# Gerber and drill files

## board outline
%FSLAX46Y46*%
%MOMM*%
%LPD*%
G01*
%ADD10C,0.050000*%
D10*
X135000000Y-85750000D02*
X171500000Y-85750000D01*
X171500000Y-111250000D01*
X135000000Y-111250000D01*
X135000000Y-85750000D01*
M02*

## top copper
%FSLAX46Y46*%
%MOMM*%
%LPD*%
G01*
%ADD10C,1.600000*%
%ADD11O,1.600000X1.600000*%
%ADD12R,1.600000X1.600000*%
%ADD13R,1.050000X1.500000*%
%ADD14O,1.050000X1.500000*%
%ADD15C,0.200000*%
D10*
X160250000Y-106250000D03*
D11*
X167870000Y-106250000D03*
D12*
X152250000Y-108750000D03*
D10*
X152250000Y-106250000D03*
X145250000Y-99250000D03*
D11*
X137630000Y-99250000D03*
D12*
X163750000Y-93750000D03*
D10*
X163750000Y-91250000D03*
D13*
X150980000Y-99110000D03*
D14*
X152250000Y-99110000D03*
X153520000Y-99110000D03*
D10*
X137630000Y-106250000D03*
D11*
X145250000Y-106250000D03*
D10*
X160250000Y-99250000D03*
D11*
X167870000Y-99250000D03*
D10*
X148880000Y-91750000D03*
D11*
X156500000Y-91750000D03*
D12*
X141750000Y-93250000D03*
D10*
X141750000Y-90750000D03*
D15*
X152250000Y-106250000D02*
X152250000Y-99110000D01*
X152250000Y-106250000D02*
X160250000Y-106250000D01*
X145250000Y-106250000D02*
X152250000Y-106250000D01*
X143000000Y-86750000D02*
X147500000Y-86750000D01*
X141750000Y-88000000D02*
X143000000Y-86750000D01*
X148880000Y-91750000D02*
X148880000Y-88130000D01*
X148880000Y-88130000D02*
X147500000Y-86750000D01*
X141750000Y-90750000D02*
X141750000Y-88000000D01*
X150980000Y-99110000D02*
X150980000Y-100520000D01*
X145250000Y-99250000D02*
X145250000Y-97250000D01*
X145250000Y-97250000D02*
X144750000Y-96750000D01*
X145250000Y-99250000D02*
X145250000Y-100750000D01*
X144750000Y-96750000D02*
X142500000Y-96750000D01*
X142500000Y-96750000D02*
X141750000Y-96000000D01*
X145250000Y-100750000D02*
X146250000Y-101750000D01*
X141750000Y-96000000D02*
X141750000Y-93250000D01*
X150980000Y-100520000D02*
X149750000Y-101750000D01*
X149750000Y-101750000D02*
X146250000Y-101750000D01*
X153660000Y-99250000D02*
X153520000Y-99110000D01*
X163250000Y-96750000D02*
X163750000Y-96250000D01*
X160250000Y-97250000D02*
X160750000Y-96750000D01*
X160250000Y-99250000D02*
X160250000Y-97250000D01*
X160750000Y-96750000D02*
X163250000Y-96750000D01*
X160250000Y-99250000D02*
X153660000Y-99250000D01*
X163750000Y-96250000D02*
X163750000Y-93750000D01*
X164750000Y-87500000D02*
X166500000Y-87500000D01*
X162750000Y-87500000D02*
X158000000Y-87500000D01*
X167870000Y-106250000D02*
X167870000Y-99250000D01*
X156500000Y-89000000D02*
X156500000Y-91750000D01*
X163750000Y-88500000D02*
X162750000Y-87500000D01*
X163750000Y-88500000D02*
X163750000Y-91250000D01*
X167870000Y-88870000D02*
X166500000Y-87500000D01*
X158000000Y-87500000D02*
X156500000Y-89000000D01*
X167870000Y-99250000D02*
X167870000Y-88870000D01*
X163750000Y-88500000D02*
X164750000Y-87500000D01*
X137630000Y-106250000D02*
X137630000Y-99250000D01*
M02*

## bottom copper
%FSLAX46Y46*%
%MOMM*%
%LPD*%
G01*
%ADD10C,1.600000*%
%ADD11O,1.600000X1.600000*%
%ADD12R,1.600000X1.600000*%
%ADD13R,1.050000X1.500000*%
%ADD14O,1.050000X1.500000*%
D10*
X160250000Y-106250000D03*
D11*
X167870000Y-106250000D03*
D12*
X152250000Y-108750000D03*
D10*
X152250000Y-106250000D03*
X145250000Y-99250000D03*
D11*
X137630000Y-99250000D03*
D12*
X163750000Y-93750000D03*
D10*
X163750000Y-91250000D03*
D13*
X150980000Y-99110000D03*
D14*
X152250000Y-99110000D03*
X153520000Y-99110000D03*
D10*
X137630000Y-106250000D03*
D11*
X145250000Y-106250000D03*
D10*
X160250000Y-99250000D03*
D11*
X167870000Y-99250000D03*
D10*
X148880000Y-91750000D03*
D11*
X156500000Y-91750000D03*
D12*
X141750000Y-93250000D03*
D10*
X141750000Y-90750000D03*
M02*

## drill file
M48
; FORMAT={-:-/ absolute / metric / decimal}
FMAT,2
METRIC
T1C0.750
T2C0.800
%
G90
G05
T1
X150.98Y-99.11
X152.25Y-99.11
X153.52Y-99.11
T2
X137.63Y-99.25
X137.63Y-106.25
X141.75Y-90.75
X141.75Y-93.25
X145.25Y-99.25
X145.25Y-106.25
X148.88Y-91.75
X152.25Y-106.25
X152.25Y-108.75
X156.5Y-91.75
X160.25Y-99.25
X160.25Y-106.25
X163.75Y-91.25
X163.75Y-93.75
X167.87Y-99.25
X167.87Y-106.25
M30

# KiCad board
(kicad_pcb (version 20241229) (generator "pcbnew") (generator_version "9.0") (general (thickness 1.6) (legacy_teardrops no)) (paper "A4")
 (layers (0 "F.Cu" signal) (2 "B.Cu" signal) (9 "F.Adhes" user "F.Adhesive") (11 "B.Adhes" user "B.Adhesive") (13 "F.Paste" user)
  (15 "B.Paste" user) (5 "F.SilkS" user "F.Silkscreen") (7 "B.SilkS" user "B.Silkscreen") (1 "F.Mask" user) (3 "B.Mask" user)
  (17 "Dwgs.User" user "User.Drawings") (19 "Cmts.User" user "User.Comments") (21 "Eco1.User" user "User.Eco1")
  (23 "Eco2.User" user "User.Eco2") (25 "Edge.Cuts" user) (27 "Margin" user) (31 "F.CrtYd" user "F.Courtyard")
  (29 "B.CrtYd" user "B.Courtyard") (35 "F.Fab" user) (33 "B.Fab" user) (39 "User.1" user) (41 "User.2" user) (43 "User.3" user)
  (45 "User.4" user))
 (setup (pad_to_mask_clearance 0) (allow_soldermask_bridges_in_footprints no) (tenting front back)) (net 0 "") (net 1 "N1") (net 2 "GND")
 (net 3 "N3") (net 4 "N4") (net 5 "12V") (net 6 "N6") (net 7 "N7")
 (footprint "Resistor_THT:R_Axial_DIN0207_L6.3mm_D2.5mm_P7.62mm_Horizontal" (layer "F.Cu") (at 160.25 106.25)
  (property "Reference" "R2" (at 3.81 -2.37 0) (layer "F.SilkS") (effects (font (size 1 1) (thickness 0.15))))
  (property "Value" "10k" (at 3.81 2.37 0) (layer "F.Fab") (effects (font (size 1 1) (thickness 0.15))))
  (pad "1" thru_hole circle (at 0 0) (size 1.6 1.6) (drill 0.8) (layers "*.Cu" "*.Mask") (remove_unused_layers no) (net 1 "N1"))
  (pad "2" thru_hole oval (at 7.62 0) (size 1.6 1.6) (drill 0.8) (layers "*.Cu" "*.Mask") (remove_unused_layers no) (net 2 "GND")))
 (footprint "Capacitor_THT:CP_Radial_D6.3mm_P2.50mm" (layer "F.Cu") (at 152.25 108.75 90)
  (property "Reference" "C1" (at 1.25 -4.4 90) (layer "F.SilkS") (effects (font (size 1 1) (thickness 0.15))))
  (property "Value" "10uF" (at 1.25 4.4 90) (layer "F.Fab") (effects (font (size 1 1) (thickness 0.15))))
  (pad "1" thru_hole rect (at 0 0 90) (size 1.6 1.6) (drill 0.8) (layers "*.Cu" "*.Mask") (remove_unused_layers no) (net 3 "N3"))
  (pad "2" thru_hole circle (at 2.5 0 90) (size 1.6 1.6) (drill 0.8) (layers "*.Cu" "*.Mask") (remove_unused_layers no) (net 1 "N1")))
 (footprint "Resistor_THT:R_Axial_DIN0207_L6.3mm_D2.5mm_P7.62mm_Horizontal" (layer "F.Cu") (at 145.25 99.25 180)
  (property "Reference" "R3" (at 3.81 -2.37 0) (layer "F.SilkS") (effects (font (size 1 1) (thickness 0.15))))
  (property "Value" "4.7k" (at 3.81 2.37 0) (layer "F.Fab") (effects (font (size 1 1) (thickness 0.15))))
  (pad "1" thru_hole circle (at 0 0 180) (size 1.6 1.6) (drill 0.8) (layers "*.Cu" "*.Mask") (remove_unused_layers no) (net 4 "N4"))
  (pad "2" thru_hole oval (at 7.62 0 180) (size 1.6 1.6) (drill 0.8) (layers "*.Cu" "*.Mask") (remove_unused_layers no) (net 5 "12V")))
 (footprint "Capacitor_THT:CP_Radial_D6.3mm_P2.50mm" (layer "F.Cu") (at 163.75 93.75 90)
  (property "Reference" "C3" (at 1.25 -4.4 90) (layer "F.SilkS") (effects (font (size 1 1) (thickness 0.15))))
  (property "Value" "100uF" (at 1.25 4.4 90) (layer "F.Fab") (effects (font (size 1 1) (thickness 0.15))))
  (pad "1" thru_hole rect (at 0 0 90) (size 1.6 1.6) (drill 0.8) (layers "*.Cu" "*.Mask") (remove_unused_layers no) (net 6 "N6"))
  (pad "2" thru_hole circle (at 2.5 0 90) (size 1.6 1.6) (drill 0.8) (layers "*.Cu" "*.Mask") (remove_unused_layers no) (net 2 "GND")))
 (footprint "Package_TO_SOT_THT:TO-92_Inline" (layer "F.Cu") (at 150.98 99.11)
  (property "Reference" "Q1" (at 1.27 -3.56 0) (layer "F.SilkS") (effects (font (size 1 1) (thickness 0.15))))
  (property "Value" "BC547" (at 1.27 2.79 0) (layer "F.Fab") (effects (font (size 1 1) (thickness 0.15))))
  (pad "1" thru_hole rect (at 0 0) (size 1.05 1.5) (drill 0.75) (layers "*.Cu" "*.Mask") (remove_unused_layers no) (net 4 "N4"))
  (pad "2" thru_hole oval (at 1.27 0) (size 1.05 1.5) (drill 0.75) (layers "*.Cu" "*.Mask") (remove_unused_layers no) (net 1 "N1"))
  (pad "3" thru_hole oval (at 2.54 0) (size 1.05 1.5) (drill 0.75) (layers "*.Cu" "*.Mask") (remove_unused_layers no) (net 6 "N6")))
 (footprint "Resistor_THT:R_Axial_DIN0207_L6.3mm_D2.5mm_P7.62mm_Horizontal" (layer "F.Cu") (at 137.63 106.25)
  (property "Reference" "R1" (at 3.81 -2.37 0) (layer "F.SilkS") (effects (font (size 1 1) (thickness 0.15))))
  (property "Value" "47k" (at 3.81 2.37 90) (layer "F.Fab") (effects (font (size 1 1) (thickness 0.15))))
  (pad "1" thru_hole circle (at 0 0) (size 1.6 1.6) (drill 0.8) (layers "*.Cu" "*.Mask") (remove_unused_layers no) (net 5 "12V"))
  (pad "2" thru_hole oval (at 7.62 0) (size 1.6 1.6) (drill 0.8) (layers "*.Cu" "*.Mask") (remove_unused_layers no) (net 1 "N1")))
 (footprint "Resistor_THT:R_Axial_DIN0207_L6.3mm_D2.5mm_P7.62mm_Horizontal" (layer "F.Cu") (at 160.25 99.25)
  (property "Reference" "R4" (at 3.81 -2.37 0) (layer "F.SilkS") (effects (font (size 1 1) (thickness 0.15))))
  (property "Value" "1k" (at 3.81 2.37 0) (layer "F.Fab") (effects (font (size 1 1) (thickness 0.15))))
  (pad "1" thru_hole circle (at 0 0) (size 1.6 1.6) (drill 0.8) (layers "*.Cu" "*.Mask") (remove_unused_layers no) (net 6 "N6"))
  (pad "2" thru_hole oval (at 7.62 0) (size 1.6 1.6) (drill 0.8) (layers "*.Cu" "*.Mask") (remove_unused_layers no) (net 2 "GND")))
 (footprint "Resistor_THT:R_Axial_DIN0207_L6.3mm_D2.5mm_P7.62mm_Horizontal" (layer "F.Cu") (at 148.88 91.75)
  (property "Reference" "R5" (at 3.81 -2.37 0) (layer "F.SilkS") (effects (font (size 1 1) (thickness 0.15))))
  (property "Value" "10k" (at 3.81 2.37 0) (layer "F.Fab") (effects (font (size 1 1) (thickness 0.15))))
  (pad "1" thru_hole circle (at 0 0) (size 1.6 1.6) (drill 0.8) (layers "*.Cu" "*.Mask") (remove_unused_layers no) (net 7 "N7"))
  (pad "2" thru_hole oval (at 7.62 0) (size 1.6 1.6) (drill 0.8) (layers "*.Cu" "*.Mask") (remove_unused_layers no) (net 2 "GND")))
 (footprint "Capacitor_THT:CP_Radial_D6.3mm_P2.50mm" (layer "F.Cu") (at 141.75 93.25 90)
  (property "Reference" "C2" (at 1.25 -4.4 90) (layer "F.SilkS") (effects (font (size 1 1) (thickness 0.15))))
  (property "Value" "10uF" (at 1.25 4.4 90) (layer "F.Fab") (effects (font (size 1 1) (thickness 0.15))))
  (pad "1" thru_hole rect (at 0 0 90) (size 1.6 1.6) (drill 0.8) (layers "*.Cu" "*.Mask") (remove_unused_layers no) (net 4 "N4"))
  (pad "2" thru_hole circle (at 2.5 0 90) (size 1.6 1.6) (drill 0.8) (layers "*.Cu" "*.Mask") (remove_unused_layers no) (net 7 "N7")))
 (gr_rect (start 135 85.75) (end 171.5 111.25) (stroke (width 0.05) (type default)) (fill no) (layer "Edge.Cuts"))
 (segment (start 152.25 106.25) (end 152.25 99.11) (width 0.2) (layer "F.Cu") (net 1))
 (segment (start 152.25 106.25) (end 160.25 106.25) (width 0.2) (layer "F.Cu") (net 1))
 (segment (start 145.25 106.25) (end 152.25 106.25) (width 0.2) (layer "F.Cu") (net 1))
 (segment (start 143 86.75) (end 147.5 86.75) (width 0.2) (layer "F.Cu") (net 7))
 (segment (start 141.75 88) (end 143 86.75) (width 0.2) (layer "F.Cu") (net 7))
 (segment (start 148.88 91.75) (end 148.88 88.13) (width 0.2) (layer "F.Cu") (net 7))
 (segment (start 148.88 88.13) (end 147.5 86.75) (width 0.2) (layer "F.Cu") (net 7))
 (segment (start 141.75 90.75) (end 141.75 88) (width 0.2) (layer "F.Cu") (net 7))
 (segment (start 150.98 99.11) (end 150.98 100.52) (width 0.2) (layer "F.Cu") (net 4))
 (segment (start 145.25 99.25) (end 145.25 97.25) (width 0.2) (layer "F.Cu") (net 4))
 (segment (start 145.25 97.25) (end 144.75 96.75) (width 0.2) (layer "F.Cu") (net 4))
 (segment (start 145.25 99.25) (end 145.25 100.75) (width 0.2) (layer "F.Cu") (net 4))
 (segment (start 144.75 96.75) (end 142.5 96.75) (width 0.2) (layer "F.Cu") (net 4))
 (segment (start 142.5 96.75) (end 141.75 96) (width 0.2) (layer "F.Cu") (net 4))
 (segment (start 145.25 100.75) (end 146.25 101.75) (width 0.2) (layer "F.Cu") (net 4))
 (segment (start 141.75 96) (end 141.75 93.25) (width 0.2) (layer "F.Cu") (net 4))
 (segment (start 150.98 100.52) (end 149.75 101.75) (width 0.2) (layer "F.Cu") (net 4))
 (segment (start 149.75 101.75) (end 146.25 101.75) (width 0.2) (layer "F.Cu") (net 4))
 (segment (start 153.66 99.25) (end 153.52 99.11) (width 0.2) (layer "F.Cu") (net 6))
 (segment (start 163.25 96.75) (end 163.75 96.25) (width 0.2) (layer "F.Cu") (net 6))
 (segment (start 160.25 97.25) (end 160.75 96.75) (width 0.2) (layer "F.Cu") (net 6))
 (segment (start 160.25 99.25) (end 160.25 97.25) (width 0.2) (layer "F.Cu") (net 6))
 (segment (start 160.75 96.75) (end 163.25 96.75) (width 0.2) (layer "F.Cu") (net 6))
 (segment (start 160.25 99.25) (end 153.66 99.25) (width 0.2) (layer "F.Cu") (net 6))
 (segment (start 163.75 96.25) (end 163.75 93.75) (width 0.2) (layer "F.Cu") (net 6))
 (segment (start 164.75 87.5) (end 166.5 87.5) (width 0.2) (layer "F.Cu") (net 2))
 (segment (start 162.75 87.5) (end 158 87.5) (width 0.2) (layer "F.Cu") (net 2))
 (segment (start 167.87 106.25) (end 167.87 99.25) (width 0.2) (layer "F.Cu") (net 2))
 (segment (start 156.5 89) (end 156.5 91.75) (width 0.2) (layer "F.Cu") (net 2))
 (segment (start 163.75 88.5) (end 162.75 87.5) (width 0.2) (layer "F.Cu") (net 2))
 (segment (start 163.75 88.5) (end 163.75 91.25) (width 0.2) (layer "F.Cu") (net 2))
 (segment (start 167.87 88.87) (end 166.5 87.5) (width 0.2) (layer "F.Cu") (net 2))
 (segment (start 158 87.5) (end 156.5 89) (width 0.2) (layer "F.Cu") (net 2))
 (segment (start 167.87 99.25) (end 167.87 88.87) (width 0.2) (layer "F.Cu") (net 2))
 (segment (start 163.75 88.5) (end 164.75 87.5) (width 0.2) (layer "F.Cu") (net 2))
 (segment (start 137.63 106.25) (end 137.63 99.25) (width 0.2) (layer "F.Cu") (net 5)))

